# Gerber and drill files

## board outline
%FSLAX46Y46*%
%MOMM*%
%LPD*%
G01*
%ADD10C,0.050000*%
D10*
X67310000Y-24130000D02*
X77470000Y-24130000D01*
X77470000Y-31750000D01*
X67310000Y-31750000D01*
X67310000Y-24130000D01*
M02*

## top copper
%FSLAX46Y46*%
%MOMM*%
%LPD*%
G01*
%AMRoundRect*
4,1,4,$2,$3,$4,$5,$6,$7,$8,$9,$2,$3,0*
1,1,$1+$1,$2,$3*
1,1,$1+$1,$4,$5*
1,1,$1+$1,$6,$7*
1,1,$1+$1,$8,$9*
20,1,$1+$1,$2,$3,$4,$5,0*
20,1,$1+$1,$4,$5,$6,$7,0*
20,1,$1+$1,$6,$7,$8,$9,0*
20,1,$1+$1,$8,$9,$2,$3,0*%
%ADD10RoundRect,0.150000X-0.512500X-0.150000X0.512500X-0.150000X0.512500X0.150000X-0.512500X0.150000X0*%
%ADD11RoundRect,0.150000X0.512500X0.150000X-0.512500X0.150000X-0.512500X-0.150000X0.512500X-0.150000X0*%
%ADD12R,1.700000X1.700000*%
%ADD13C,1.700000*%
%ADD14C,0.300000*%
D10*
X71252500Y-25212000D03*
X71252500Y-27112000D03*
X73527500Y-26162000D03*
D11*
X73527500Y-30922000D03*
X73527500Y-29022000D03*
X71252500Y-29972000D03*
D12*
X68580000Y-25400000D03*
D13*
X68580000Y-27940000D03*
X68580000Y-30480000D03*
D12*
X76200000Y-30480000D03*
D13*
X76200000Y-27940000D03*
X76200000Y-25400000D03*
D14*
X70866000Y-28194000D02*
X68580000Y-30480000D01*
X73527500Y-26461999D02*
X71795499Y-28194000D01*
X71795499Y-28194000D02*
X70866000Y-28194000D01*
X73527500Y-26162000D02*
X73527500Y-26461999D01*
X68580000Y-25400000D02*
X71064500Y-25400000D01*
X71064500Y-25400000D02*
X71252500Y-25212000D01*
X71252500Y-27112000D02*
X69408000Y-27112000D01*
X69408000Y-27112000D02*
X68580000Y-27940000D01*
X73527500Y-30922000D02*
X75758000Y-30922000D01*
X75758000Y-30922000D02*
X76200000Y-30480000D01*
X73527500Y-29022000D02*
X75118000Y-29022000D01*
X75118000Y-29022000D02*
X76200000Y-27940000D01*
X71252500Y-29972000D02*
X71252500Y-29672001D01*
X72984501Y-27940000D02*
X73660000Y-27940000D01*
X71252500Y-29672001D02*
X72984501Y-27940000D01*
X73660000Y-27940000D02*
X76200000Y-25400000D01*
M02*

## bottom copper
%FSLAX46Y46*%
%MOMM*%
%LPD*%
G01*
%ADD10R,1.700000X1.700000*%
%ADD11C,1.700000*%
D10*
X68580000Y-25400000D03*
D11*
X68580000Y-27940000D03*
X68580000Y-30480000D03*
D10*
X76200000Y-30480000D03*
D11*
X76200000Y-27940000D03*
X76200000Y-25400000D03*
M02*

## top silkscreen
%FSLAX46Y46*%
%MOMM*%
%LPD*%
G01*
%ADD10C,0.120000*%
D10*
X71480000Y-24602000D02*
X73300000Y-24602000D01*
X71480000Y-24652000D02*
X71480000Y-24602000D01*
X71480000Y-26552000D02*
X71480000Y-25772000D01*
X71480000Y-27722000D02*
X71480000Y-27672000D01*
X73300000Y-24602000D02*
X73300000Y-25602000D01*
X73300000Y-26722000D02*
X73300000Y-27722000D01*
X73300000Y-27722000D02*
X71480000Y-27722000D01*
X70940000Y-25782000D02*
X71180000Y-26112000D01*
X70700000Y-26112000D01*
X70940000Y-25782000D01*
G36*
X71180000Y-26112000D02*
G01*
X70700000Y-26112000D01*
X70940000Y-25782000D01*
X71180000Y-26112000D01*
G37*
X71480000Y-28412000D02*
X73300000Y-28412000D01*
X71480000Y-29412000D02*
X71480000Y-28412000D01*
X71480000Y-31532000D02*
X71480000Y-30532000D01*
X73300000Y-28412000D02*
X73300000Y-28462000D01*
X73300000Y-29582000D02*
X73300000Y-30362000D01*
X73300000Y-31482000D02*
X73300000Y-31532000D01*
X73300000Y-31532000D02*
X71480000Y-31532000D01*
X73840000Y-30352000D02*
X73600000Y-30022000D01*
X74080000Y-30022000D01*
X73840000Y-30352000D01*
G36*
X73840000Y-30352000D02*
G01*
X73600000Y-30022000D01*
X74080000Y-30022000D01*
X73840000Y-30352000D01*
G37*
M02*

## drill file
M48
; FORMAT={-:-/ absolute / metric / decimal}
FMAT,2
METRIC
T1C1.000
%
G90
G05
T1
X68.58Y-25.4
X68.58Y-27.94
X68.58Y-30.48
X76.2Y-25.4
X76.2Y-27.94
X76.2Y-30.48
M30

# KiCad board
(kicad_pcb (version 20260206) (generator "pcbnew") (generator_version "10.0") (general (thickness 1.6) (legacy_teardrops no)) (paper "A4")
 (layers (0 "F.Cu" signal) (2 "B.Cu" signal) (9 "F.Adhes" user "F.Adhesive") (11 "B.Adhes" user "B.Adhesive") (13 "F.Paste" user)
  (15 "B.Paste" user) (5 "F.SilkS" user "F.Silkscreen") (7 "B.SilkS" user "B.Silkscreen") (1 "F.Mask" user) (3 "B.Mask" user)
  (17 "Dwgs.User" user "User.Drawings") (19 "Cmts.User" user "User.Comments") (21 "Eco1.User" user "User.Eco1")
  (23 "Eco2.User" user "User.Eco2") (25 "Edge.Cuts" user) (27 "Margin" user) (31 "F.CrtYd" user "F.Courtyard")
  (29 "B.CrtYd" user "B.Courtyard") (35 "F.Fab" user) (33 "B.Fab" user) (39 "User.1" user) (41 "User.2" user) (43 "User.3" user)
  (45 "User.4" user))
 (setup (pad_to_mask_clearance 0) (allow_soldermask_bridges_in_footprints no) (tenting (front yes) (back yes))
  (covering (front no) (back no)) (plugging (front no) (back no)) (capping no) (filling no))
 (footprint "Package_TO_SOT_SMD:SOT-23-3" (layer "F.Cu") (at 72.39 26.162)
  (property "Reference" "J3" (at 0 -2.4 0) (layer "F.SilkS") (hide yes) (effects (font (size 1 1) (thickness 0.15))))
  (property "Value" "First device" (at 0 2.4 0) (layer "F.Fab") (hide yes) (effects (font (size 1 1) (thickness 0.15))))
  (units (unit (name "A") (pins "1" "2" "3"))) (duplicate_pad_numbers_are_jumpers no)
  (fp_line (start -0.91 -1.56) (end 0.91 -1.56) (stroke (width 0.12) (type solid)) (layer "F.SilkS"))
  (fp_line (start -0.91 -1.51) (end -0.91 -1.56) (stroke (width 0.12) (type solid)) (layer "F.SilkS"))
  (fp_line (start -0.91 0.39) (end -0.91 -0.39) (stroke (width 0.12) (type solid)) (layer "F.SilkS"))
  (fp_line (start -0.91 1.56) (end -0.91 1.51) (stroke (width 0.12) (type solid)) (layer "F.SilkS"))
  (fp_line (start 0.91 -1.56) (end 0.91 -0.56) (stroke (width 0.12) (type solid)) (layer "F.SilkS"))
  (fp_line (start 0.91 0.56) (end 0.91 1.56) (stroke (width 0.12) (type solid)) (layer "F.SilkS"))
  (fp_line (start 0.91 1.56) (end -0.91 1.56) (stroke (width 0.12) (type solid)) (layer "F.SilkS"))
  (fp_poly (pts (xy -1.45 -0.38) (xy -1.21 -0.05) (xy -1.69 -0.05)) (stroke (width 0.12) (type solid)) (fill yes) (layer "F.SilkS"))
  (pad "1" smd roundrect (at -1.1375 -0.95) (size 1.325 0.6) (layers "F.Cu" "F.Mask" "F.Paste") (roundrect_rratio 0.25)
   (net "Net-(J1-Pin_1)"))
  (pad "2" smd roundrect (at -1.1375 0.95) (size 1.325 0.6) (layers "F.Cu" "F.Mask" "F.Paste") (roundrect_rratio 0.25)
   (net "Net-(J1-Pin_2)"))
  (pad "3" smd roundrect (at 1.1375 0) (size 1.325 0.6) (layers "F.Cu" "F.Mask" "F.Paste") (roundrect_rratio 0.25) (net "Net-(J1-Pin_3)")))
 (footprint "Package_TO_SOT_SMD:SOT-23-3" (layer "F.Cu") (at 72.39 29.972 180)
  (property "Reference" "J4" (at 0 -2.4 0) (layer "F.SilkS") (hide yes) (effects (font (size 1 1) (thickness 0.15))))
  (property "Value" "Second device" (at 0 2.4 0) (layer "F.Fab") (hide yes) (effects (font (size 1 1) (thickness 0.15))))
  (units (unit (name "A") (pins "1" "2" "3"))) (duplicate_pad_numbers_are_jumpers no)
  (fp_line (start 0.91 1.56) (end -0.91 1.56) (stroke (width 0.12) (type solid)) (layer "F.SilkS"))
  (fp_line (start 0.91 0.56) (end 0.91 1.56) (stroke (width 0.12) (type solid)) (layer "F.SilkS"))
  (fp_line (start 0.91 -1.56) (end 0.91 -0.56) (stroke (width 0.12) (type solid)) (layer "F.SilkS"))
  (fp_line (start -0.91 1.56) (end -0.91 1.51) (stroke (width 0.12) (type solid)) (layer "F.SilkS"))
  (fp_line (start -0.91 0.39) (end -0.91 -0.39) (stroke (width 0.12) (type solid)) (layer "F.SilkS"))
  (fp_line (start -0.91 -1.51) (end -0.91 -1.56) (stroke (width 0.12) (type solid)) (layer "F.SilkS"))
  (fp_line (start -0.91 -1.56) (end 0.91 -1.56) (stroke (width 0.12) (type solid)) (layer "F.SilkS"))
  (fp_poly (pts (xy -1.45 -0.38) (xy -1.21 -0.05) (xy -1.69 -0.05)) (stroke (width 0.12) (type solid)) (fill yes) (layer "F.SilkS"))
  (pad "1" smd roundrect (at -1.1375 -0.95 180) (size 1.325 0.6) (layers "F.Cu" "F.Mask" "F.Paste") (roundrect_rratio 0.25)
   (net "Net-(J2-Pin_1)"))
  (pad "2" smd roundrect (at -1.1375 0.95 180) (size 1.325 0.6) (layers "F.Cu" "F.Mask" "F.Paste") (roundrect_rratio 0.25)
   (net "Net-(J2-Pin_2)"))
  (pad "3" smd roundrect (at 1.1375 0 180) (size 1.325 0.6) (layers "F.Cu" "F.Mask" "F.Paste") (roundrect_rratio 0.25)
   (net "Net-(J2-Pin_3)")))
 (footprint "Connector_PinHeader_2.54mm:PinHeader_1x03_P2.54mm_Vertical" (layer "B.Cu") (at 68.58 25.4 180)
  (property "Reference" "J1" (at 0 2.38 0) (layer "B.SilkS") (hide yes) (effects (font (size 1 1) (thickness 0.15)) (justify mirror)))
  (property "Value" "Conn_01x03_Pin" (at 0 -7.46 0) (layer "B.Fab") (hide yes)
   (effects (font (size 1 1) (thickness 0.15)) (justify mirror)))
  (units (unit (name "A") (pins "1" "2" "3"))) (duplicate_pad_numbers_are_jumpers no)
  (pad "1" thru_hole rect (at 0 0 180) (size 1.7 1.7) (drill 1) (layers "*.Cu" "*.Mask") (remove_unused_layers no) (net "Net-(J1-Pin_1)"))
  (pad "2" thru_hole circle (at 0 -2.54 180) (size 1.7 1.7) (drill 1) (layers "*.Cu" "*.Mask") (remove_unused_layers no)
   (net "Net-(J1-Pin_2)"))
  (pad "3" thru_hole circle (at 0 -5.08 180) (size 1.7 1.7) (drill 1) (layers "*.Cu" "*.Mask") (remove_unused_layers no)
   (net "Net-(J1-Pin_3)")))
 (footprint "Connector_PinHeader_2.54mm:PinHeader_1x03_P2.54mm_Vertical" (layer "B.Cu") (at 76.2 30.48)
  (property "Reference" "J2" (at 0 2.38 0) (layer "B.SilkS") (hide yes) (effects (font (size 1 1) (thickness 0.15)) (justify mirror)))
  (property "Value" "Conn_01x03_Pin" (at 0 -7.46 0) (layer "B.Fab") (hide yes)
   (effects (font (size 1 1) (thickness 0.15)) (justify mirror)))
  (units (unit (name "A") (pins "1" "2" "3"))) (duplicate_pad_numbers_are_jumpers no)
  (pad "1" thru_hole rect (at 0 0) (size 1.7 1.7) (drill 1) (layers "*.Cu" "*.Mask") (remove_unused_layers no) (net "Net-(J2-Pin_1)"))
  (pad "2" thru_hole circle (at 0 -2.54) (size 1.7 1.7) (drill 1) (layers "*.Cu" "*.Mask") (remove_unused_layers no) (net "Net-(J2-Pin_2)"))
  (pad "3" thru_hole circle (at 0 -5.08) (size 1.7 1.7) (drill 1) (layers "*.Cu" "*.Mask") (remove_unused_layers no) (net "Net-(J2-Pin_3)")))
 (gr_rect (start 67.31 24.13) (end 77.47 31.75) (stroke (width 0.05) (type default)) (fill no) (layer "Edge.Cuts"))
 (segment (start 70.866 28.194) (end 68.58 30.48) (width 0.3) (layer "F.Cu") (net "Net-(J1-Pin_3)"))
 (segment (start 73.5275 26.461999) (end 71.795499 28.194) (width 0.3) (layer "F.Cu") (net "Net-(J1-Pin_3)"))
 (segment (start 71.795499 28.194) (end 70.866 28.194) (width 0.3) (layer "F.Cu") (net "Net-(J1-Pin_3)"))
 (segment (start 73.5275 26.162) (end 73.5275 26.461999) (width 0.3) (layer "F.Cu") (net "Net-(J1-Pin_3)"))
 (segment (start 68.58 25.4) (end 71.0645 25.4) (width 0.3) (layer "F.Cu") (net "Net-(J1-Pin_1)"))
 (segment (start 71.0645 25.4) (end 71.2525 25.212) (width 0.3) (layer "F.Cu") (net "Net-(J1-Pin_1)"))
 (segment (start 71.2525 27.112) (end 69.408 27.112) (width 0.3) (layer "F.Cu") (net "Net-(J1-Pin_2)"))
 (segment (start 69.408 27.112) (end 68.58 27.94) (width 0.3) (layer "F.Cu") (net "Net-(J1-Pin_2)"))
 (segment (start 73.5275 30.922) (end 75.758 30.922) (width 0.3) (layer "F.Cu") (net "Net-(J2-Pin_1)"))
 (segment (start 75.758 30.922) (end 76.2 30.48) (width 0.3) (layer "F.Cu") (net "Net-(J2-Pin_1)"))
 (segment (start 73.5275 29.022) (end 75.118 29.022) (width 0.3) (layer "F.Cu") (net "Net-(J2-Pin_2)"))
 (segment (start 75.118 29.022) (end 76.2 27.94) (width 0.3) (layer "F.Cu") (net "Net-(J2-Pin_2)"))
 (segment (start 71.2525 29.972) (end 71.2525 29.672001) (width 0.3) (layer "F.Cu") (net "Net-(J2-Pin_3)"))
 (segment (start 72.984501 27.94) (end 73.66 27.94) (width 0.3) (layer "F.Cu") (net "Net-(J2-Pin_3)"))
 (segment (start 71.2525 29.672001) (end 72.984501 27.94) (width 0.3) (layer "F.Cu") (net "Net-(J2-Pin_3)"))
 (segment (start 73.66 27.94) (end 76.2 25.4) (width 0.3) (layer "F.Cu") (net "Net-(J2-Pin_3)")))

